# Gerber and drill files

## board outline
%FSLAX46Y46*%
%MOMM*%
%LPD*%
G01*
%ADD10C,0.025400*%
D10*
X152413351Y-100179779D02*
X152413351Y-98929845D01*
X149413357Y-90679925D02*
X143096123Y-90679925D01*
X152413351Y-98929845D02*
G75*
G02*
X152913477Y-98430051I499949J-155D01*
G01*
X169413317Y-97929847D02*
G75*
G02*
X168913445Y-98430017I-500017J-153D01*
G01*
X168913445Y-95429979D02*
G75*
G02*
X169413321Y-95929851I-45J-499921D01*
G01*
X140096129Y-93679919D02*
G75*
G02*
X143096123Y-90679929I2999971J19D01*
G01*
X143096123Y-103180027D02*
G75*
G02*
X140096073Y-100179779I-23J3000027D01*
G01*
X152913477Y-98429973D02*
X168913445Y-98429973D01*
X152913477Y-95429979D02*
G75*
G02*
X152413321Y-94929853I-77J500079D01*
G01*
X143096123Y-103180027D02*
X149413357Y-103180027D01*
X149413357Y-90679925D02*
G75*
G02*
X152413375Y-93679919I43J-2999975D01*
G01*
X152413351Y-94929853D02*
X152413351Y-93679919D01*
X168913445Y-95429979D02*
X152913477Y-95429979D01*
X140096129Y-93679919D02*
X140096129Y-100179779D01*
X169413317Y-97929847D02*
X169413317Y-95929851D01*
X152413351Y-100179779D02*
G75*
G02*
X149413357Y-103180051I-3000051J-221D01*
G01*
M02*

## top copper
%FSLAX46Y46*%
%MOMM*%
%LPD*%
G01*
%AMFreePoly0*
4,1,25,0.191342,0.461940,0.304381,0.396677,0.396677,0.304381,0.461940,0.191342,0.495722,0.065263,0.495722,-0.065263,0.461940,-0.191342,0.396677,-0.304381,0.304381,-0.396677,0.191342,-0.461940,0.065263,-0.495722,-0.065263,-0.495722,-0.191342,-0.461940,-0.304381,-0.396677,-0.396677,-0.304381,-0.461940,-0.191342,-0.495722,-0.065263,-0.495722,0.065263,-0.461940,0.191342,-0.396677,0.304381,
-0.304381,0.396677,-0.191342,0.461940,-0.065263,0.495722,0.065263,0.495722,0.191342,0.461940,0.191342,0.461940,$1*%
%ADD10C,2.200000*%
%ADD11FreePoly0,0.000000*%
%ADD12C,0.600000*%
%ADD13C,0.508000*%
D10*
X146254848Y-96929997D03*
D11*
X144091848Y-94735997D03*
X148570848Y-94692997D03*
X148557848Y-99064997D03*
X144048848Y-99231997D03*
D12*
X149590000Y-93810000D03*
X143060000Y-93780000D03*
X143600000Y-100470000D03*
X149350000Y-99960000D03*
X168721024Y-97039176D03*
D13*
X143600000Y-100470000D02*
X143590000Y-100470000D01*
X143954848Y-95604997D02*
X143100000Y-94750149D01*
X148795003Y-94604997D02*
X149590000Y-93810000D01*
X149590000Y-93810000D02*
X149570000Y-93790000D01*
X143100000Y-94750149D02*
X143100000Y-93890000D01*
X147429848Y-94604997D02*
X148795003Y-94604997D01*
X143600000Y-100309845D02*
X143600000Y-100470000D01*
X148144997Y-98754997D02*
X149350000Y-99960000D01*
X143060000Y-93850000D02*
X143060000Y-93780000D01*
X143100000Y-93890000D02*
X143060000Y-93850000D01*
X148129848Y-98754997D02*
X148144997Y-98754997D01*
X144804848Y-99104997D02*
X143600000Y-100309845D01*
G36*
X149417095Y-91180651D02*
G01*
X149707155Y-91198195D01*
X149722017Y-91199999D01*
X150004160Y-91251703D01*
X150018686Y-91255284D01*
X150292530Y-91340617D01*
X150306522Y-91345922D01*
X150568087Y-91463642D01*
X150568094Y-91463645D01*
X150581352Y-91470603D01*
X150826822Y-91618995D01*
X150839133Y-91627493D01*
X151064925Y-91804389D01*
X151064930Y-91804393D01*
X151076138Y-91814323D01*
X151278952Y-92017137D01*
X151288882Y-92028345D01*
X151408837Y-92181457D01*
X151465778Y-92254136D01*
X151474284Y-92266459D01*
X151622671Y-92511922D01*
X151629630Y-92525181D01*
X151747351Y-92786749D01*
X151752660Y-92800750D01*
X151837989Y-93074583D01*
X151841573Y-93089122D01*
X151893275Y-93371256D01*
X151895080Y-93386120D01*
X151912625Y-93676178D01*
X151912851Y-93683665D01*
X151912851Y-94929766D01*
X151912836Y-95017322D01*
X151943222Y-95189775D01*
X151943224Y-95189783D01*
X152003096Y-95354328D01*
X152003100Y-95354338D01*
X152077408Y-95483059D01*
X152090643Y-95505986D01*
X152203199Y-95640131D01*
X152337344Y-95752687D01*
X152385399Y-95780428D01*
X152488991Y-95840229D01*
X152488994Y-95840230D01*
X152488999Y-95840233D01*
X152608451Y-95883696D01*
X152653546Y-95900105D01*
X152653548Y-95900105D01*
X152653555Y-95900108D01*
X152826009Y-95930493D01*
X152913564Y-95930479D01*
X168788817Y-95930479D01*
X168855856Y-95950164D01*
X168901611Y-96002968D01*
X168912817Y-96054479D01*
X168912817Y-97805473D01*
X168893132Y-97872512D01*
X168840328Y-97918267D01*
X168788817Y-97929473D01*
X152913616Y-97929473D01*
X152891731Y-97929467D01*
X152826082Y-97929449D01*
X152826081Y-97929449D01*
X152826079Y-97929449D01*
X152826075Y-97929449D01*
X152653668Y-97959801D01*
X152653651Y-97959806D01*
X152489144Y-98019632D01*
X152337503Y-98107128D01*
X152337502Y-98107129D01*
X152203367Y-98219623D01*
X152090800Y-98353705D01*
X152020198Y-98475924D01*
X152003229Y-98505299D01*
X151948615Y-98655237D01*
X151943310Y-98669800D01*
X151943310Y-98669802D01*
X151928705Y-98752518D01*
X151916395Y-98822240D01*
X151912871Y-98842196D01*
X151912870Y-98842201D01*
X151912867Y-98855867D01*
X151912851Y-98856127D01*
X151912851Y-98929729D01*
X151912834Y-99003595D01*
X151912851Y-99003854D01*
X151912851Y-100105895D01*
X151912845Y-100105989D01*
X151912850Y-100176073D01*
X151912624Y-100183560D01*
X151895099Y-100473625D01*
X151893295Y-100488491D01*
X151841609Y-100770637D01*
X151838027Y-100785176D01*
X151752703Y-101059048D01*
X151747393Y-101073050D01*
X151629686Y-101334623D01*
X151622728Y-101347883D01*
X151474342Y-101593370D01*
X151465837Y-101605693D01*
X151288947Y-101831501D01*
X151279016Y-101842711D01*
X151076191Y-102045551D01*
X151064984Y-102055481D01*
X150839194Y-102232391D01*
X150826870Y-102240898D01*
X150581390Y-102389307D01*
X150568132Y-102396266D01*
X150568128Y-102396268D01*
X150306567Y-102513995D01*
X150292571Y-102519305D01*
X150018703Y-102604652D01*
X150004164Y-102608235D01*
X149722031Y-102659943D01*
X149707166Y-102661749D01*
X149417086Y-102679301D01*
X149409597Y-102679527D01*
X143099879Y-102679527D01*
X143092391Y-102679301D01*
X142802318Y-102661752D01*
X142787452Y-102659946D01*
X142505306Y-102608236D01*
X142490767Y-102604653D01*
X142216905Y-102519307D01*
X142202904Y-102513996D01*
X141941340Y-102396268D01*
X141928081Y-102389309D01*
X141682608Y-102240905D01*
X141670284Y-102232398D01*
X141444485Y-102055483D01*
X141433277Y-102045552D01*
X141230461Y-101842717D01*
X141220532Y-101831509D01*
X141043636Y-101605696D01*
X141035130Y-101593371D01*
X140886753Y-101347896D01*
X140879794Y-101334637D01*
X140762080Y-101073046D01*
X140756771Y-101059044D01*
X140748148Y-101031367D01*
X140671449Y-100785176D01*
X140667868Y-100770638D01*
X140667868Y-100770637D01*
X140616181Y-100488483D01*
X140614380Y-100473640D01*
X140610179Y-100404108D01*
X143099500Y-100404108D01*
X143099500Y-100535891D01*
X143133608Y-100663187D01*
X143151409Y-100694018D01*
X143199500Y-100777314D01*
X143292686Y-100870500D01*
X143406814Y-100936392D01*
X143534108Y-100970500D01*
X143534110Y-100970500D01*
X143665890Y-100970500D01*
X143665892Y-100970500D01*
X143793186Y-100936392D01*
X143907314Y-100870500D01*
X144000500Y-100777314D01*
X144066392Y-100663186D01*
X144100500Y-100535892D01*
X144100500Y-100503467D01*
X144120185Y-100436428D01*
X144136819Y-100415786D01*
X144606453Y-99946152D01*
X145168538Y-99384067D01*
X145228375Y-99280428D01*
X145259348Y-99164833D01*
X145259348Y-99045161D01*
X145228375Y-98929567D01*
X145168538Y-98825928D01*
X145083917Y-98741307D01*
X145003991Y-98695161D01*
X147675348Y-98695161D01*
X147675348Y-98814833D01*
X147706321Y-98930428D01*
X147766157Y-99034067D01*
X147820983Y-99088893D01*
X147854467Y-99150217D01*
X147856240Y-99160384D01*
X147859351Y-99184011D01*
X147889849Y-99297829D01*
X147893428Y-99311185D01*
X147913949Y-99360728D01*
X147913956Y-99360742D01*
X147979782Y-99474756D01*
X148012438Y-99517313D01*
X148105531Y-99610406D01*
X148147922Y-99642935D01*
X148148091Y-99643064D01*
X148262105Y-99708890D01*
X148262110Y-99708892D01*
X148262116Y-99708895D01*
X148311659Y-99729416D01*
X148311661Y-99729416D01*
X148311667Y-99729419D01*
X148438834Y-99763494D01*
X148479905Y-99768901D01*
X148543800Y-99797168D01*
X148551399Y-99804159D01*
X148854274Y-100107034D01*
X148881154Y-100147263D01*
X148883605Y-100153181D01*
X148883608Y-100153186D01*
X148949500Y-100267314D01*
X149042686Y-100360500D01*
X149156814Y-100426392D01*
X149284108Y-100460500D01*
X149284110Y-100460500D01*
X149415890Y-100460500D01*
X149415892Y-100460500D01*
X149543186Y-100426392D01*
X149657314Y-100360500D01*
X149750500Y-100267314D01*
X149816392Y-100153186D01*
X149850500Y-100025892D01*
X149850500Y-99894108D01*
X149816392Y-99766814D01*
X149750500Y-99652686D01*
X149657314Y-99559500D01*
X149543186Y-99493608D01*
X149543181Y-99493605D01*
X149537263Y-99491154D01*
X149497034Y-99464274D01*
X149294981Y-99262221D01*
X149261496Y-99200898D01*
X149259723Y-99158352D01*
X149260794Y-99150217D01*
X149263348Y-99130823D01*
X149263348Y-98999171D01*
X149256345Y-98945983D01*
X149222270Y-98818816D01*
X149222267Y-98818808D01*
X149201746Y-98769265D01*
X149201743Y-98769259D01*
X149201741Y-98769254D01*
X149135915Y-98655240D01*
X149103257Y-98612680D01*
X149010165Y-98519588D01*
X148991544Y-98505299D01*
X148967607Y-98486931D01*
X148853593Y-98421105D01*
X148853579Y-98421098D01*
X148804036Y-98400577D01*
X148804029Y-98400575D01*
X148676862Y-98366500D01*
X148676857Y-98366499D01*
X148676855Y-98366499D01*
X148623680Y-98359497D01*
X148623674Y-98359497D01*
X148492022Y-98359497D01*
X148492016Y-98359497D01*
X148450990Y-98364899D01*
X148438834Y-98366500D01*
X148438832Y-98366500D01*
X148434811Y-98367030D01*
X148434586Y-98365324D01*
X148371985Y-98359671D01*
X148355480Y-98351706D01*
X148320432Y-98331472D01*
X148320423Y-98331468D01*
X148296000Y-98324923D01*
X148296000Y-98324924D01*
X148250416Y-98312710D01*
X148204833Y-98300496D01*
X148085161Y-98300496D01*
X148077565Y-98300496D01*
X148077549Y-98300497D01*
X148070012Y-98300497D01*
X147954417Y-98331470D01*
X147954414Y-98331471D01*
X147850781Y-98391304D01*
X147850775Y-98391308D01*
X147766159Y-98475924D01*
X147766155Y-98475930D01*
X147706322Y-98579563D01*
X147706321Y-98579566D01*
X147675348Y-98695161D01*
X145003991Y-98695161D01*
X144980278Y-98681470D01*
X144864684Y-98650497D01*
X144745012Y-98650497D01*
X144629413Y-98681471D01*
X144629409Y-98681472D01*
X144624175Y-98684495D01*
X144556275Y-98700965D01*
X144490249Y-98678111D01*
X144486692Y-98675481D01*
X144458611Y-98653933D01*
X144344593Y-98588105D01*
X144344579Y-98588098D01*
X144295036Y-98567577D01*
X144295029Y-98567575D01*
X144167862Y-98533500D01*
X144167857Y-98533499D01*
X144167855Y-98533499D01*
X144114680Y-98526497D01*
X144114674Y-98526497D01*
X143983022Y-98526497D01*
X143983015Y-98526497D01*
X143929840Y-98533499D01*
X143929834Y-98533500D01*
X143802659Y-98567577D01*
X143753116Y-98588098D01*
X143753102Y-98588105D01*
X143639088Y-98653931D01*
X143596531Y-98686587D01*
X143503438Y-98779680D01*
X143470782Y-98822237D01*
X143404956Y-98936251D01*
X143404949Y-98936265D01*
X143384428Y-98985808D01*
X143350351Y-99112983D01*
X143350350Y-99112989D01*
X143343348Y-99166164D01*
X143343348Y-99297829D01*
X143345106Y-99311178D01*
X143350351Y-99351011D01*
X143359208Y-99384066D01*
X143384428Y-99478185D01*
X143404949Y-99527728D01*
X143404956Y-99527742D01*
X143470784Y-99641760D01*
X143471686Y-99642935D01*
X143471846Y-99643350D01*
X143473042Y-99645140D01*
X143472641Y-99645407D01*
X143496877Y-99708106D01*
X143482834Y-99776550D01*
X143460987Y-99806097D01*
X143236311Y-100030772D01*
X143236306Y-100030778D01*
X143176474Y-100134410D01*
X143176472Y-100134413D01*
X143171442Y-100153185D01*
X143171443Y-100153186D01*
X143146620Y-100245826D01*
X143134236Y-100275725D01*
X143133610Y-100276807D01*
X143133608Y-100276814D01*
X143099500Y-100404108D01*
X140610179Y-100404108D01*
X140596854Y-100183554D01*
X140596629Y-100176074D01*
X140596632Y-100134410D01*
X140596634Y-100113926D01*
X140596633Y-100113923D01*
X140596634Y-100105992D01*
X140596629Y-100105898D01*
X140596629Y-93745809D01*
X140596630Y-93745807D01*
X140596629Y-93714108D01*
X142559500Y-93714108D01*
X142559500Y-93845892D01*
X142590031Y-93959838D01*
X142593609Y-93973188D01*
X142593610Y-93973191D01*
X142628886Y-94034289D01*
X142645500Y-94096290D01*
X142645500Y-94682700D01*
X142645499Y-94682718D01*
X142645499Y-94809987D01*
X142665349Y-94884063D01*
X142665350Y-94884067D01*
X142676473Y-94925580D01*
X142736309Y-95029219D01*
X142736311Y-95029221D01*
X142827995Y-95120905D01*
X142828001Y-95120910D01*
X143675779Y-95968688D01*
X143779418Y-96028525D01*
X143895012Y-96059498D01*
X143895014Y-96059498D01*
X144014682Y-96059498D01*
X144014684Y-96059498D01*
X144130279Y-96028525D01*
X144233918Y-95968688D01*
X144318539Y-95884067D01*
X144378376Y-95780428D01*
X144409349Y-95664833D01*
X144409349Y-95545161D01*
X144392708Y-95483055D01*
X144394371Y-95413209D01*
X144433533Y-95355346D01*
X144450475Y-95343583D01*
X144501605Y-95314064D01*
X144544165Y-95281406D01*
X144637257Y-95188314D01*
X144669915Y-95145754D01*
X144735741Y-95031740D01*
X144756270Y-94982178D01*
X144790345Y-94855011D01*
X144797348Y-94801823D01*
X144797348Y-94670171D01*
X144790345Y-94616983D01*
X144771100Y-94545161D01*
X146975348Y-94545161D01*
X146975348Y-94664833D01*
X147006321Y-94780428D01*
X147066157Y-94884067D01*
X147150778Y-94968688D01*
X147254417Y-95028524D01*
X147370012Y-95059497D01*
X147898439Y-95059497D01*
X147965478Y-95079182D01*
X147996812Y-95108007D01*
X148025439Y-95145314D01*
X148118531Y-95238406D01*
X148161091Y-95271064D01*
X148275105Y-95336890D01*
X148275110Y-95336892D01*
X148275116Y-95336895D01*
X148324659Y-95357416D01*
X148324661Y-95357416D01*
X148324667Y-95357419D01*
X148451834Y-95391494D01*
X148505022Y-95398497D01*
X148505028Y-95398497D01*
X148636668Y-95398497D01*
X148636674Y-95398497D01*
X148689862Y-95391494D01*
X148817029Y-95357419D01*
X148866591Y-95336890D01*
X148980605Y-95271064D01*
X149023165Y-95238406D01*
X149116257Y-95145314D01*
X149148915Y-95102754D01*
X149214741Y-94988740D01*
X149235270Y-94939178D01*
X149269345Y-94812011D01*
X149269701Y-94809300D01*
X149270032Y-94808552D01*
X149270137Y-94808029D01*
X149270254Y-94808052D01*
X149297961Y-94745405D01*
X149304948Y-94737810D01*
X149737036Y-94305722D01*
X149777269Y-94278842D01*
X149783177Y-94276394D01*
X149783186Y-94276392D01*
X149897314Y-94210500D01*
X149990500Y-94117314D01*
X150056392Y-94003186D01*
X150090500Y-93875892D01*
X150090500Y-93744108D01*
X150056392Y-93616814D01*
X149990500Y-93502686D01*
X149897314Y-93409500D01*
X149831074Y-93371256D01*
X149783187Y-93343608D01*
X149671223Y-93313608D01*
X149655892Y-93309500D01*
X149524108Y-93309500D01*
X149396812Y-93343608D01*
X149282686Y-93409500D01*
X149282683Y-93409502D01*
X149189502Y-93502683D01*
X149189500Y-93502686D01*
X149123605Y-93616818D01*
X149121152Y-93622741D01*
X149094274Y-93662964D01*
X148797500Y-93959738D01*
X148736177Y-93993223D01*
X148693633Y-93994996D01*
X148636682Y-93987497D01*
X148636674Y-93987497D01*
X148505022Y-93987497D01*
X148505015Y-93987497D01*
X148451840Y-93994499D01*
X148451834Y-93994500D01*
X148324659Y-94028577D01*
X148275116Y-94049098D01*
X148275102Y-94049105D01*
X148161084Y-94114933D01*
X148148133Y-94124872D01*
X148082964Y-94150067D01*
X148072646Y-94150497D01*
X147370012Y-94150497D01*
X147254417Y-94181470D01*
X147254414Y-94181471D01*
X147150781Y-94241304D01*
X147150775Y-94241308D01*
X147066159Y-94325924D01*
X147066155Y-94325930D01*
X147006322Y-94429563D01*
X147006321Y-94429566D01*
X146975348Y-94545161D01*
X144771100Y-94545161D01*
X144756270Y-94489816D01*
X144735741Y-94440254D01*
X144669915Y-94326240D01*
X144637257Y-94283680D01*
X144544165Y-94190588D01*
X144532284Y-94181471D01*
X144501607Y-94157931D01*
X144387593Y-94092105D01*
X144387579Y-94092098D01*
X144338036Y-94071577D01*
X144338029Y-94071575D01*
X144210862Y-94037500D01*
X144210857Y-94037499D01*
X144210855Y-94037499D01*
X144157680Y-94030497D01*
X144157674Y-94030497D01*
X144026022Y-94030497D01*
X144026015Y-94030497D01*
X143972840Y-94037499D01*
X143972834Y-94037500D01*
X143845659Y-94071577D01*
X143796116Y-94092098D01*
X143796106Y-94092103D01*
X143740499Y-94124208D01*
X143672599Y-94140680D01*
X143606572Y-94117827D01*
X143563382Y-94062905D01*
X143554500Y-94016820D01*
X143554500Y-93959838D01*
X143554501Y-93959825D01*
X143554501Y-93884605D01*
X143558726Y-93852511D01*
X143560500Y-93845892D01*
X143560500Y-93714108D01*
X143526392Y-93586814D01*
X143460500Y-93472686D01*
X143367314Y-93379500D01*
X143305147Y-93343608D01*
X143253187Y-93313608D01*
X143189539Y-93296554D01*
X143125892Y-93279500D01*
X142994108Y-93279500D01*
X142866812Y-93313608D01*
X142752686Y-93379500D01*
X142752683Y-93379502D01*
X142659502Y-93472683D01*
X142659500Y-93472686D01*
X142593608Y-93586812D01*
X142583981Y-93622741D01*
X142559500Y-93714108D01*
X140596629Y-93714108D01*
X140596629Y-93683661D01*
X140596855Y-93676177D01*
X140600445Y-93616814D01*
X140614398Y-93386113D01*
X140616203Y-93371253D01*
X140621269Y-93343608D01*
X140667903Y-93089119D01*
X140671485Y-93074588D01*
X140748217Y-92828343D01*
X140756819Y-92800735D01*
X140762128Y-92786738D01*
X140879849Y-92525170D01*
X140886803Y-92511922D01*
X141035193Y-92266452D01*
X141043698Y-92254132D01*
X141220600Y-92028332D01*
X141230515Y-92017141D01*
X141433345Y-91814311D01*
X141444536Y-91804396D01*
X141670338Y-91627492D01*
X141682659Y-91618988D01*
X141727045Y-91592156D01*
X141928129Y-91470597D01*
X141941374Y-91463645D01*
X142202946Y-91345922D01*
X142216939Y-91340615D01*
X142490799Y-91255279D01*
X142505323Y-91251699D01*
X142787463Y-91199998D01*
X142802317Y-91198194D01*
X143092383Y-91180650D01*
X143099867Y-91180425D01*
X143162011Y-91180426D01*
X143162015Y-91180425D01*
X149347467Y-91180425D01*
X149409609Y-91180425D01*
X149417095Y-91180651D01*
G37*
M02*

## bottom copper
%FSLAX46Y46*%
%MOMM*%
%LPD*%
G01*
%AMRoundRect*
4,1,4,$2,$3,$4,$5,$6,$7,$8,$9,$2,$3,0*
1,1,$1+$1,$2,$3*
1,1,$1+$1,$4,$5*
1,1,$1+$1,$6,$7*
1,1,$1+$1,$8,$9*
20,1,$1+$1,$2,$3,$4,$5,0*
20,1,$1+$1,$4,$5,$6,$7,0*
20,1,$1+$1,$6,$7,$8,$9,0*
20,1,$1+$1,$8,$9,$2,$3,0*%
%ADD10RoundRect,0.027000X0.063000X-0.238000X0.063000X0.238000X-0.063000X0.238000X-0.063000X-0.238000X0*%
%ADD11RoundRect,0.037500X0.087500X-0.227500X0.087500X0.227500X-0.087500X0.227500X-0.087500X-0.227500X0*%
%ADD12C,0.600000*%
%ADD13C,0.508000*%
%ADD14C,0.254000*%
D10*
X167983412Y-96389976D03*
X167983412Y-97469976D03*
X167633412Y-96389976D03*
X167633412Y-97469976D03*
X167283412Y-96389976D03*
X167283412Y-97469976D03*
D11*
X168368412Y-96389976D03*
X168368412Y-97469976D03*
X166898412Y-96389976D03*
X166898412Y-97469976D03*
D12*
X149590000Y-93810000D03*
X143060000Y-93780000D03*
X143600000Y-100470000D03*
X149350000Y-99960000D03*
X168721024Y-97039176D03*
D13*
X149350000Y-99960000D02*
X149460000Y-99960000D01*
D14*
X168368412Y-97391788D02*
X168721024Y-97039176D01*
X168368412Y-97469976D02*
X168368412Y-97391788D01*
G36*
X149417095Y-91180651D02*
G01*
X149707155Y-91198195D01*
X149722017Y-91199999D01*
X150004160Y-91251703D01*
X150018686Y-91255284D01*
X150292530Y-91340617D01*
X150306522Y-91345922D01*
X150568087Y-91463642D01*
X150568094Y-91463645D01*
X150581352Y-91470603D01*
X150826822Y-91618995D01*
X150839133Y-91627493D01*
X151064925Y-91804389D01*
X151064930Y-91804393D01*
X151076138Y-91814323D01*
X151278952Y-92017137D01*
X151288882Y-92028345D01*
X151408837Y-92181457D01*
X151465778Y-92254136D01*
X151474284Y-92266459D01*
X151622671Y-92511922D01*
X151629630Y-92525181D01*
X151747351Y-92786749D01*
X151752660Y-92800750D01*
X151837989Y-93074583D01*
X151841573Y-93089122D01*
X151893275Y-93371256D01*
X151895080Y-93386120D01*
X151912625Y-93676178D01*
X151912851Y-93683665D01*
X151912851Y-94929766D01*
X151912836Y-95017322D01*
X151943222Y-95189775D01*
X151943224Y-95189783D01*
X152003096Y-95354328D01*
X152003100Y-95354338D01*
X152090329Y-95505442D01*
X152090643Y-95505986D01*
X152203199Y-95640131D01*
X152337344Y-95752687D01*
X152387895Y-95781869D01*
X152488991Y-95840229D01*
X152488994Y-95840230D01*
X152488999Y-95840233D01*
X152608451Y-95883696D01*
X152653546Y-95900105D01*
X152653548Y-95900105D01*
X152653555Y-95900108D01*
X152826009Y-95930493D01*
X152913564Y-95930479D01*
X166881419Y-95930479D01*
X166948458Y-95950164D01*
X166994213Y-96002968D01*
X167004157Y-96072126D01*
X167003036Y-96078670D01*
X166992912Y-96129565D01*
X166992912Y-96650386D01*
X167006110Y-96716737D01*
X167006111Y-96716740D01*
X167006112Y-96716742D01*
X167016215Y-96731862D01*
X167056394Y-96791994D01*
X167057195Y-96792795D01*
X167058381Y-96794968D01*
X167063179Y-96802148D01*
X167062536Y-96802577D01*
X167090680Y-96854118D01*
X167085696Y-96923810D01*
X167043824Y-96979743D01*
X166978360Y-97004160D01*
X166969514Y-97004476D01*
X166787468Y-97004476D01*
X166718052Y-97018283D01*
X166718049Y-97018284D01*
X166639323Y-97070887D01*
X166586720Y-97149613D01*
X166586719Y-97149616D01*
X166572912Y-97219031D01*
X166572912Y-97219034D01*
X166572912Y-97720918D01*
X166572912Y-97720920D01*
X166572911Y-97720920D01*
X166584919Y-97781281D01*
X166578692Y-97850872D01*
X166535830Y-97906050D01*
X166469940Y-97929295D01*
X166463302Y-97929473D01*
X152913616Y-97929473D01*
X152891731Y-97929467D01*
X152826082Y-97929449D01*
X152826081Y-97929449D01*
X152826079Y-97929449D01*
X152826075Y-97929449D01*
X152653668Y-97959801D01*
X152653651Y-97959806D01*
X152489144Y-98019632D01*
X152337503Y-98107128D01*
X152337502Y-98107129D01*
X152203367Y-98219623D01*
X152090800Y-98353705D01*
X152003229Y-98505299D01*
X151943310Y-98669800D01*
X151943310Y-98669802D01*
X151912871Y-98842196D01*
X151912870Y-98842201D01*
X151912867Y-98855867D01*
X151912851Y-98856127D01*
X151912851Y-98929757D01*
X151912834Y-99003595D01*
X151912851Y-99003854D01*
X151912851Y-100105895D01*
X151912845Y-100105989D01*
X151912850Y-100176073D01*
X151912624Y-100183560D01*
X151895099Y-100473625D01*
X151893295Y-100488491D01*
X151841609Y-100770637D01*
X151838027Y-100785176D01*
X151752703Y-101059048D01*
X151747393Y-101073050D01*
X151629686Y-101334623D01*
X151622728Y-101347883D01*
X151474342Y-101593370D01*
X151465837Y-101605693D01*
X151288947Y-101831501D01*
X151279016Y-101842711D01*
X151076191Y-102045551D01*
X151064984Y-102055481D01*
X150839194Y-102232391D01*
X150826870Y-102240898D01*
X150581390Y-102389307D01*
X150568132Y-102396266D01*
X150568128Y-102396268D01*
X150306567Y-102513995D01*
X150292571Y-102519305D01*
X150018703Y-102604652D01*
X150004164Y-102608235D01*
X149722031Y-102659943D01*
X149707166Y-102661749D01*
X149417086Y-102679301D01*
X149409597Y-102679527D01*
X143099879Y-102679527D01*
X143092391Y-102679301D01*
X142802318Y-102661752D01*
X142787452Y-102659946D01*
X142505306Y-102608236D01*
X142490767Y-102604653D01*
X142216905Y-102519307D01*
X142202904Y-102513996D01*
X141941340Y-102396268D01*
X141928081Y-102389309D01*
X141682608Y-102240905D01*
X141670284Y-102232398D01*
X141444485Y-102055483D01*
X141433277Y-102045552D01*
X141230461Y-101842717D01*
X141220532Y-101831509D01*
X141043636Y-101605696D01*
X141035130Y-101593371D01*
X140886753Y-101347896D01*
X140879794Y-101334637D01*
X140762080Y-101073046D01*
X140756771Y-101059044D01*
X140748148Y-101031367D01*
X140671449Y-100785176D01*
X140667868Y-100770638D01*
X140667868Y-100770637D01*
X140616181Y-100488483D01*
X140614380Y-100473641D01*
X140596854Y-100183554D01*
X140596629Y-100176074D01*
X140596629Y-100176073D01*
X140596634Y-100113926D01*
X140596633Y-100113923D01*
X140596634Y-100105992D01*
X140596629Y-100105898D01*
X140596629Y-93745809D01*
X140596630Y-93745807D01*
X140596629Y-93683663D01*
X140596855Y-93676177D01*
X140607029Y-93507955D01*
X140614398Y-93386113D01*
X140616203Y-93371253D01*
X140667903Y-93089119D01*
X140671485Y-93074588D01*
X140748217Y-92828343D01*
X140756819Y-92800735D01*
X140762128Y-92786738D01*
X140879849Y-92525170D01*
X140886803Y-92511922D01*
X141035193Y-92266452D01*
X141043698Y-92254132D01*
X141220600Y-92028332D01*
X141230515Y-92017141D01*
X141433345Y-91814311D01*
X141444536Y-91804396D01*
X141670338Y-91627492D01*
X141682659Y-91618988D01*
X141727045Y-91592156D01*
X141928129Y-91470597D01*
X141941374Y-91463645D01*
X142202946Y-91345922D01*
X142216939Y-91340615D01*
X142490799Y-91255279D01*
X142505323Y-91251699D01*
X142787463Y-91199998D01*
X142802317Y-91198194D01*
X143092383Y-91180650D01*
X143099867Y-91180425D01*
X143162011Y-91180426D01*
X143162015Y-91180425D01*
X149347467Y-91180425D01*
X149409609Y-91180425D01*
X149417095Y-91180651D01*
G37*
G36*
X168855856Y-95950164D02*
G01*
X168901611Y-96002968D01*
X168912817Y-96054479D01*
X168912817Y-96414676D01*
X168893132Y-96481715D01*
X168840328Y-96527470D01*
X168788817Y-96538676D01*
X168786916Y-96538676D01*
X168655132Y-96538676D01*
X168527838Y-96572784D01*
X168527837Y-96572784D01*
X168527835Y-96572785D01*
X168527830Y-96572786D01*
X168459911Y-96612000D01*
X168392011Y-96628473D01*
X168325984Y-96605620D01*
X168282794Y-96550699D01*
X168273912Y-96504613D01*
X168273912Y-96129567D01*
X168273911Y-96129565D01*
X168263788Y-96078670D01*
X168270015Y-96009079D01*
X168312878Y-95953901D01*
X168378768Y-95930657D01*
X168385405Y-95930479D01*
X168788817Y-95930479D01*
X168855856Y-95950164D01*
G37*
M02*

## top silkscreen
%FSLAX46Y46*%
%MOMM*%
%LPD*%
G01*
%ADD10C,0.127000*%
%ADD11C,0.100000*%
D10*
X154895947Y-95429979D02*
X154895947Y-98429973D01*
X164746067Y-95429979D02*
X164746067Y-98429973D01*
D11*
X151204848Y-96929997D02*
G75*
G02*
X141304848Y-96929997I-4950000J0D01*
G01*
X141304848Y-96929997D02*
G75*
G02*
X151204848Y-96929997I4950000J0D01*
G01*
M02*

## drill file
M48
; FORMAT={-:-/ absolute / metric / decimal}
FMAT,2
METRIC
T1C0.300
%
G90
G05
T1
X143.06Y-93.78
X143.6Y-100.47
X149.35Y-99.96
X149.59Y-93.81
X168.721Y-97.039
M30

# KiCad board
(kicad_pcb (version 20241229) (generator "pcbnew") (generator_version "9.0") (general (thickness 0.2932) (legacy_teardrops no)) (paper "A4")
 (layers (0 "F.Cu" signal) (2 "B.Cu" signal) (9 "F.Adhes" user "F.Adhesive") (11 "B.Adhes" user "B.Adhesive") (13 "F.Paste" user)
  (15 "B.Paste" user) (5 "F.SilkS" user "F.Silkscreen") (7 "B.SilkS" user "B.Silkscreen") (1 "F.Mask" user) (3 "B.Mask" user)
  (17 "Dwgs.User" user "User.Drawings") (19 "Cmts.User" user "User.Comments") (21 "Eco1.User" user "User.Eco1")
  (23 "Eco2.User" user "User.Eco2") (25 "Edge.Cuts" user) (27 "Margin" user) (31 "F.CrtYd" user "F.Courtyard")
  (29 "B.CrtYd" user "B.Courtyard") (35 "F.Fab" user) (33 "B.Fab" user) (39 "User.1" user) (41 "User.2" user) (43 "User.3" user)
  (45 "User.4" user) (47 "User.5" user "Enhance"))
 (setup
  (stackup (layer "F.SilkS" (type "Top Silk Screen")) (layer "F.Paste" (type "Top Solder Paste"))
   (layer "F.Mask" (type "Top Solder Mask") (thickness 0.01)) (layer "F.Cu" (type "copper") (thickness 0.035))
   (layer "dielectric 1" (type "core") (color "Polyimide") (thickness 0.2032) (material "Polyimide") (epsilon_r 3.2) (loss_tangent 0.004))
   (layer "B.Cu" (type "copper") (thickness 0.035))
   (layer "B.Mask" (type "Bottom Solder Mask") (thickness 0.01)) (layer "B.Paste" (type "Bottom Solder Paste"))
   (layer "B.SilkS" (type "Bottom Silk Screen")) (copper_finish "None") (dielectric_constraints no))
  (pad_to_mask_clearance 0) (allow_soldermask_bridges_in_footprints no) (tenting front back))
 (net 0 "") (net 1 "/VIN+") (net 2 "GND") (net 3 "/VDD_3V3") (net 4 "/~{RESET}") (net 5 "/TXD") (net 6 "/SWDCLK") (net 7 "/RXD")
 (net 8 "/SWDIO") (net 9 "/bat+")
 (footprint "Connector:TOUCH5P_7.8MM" (layer "F.Cu") (at 146.254848 96.929997)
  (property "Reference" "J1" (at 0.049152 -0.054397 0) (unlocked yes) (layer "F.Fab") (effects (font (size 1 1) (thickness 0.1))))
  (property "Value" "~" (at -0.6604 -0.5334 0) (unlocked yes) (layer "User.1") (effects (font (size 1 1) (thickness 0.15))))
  (fp_circle (center 0 0) (end 4.95 0) (stroke (width 0.1) (type default)) (fill no) (layer "F.SilkS"))
  (pad "1" smd circle (at 0 0) (size 2.2 2.2) (layers "F.Cu" "F.Mask" "F.Paste") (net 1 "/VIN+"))
  (pad "2" smd custom (at -2.163 -2.194) (size 1 1) (layers "F.Cu" "F.Mask" "F.Paste") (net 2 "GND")
   (options (clearance outline) (anchor circle)) (primitives))
  (pad "3" smd custom (at 2.316 -2.237) (size 1 2.2) (layers "F.Cu" "F.Mask" "F.Paste") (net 2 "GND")
   (options (clearance outline) (anchor circle)) (primitives))
  (pad "4" smd custom (at 2.303 2.135) (size 1 1) (layers "F.Cu" "F.Mask" "F.Paste") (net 2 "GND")
   (options (clearance outline) (anchor circle)) (primitives))
  (pad "5" smd custom (at -2.206 2.302) (size 1 1) (layers "F.Cu" "F.Mask" "F.Paste") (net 2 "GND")
   (options (clearance outline) (anchor circle)) (primitives)))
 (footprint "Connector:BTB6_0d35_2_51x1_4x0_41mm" (layer "B.Cu") (at 167.633412 96.929976 180)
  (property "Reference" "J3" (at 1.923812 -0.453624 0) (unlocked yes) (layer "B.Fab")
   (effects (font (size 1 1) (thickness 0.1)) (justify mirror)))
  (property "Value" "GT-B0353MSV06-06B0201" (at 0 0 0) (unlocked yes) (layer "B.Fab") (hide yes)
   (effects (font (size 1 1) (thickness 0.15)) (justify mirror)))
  (pad "1" smd roundrect (at -0.35 0.54 90) (size 0.53 0.18) (layers "B.Cu" "B.Mask" "B.Paste") (roundrect_rratio 0.15) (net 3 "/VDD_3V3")
   (thermal_bridge_angle 45))
  (pad "2" smd roundrect (at -0.35 -0.54 90) (size 0.53 0.18) (layers "B.Cu" "B.Mask" "B.Paste") (roundrect_rratio 0.15) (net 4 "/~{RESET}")
   (thermal_bridge_angle 45))
  (pad "3" smd roundrect (at 0 0.54 90) (size 0.53 0.18) (layers "B.Cu" "B.Mask" "B.Paste") (roundrect_rratio 0.15) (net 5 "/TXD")
   (thermal_bridge_angle 45))
  (pad "4" smd roundrect (at 0 -0.54 90) (size 0.53 0.18) (layers "B.Cu" "B.Mask" "B.Paste") (roundrect_rratio 0.15) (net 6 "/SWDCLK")
   (thermal_bridge_angle 45))
  (pad "5" smd roundrect (at 0.35 0.54 90) (size 0.53 0.18) (layers "B.Cu" "B.Mask" "B.Paste") (roundrect_rratio 0.15) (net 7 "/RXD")
   (thermal_bridge_angle 45))
  (pad "6" smd roundrect (at 0.35 -0.54 90) (size 0.53 0.18) (layers "B.Cu" "B.Mask" "B.Paste") (roundrect_rratio 0.15) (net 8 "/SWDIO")
   (thermal_bridge_angle 45))
  (pad "S1" smd roundrect (at -0.735 0.54 90) (size 0.53 0.25) (layers "B.Cu" "B.Mask" "B.Paste") (roundrect_rratio 0.15) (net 2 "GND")
   (thermal_bridge_angle 45))
  (pad "S2" smd roundrect (at -0.735 -0.54 90) (size 0.53 0.25) (layers "B.Cu" "B.Mask" "B.Paste") (roundrect_rratio 0.15) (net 1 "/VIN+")
   (thermal_bridge_angle 45))
  (pad "S3" smd roundrect (at 0.735 0.54 90) (size 0.53 0.25) (layers "B.Cu" "B.Mask" "B.Paste") (roundrect_rratio 0.15) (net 2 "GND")
   (thermal_bridge_angle 45))
  (pad "S4" smd roundrect (at 0.735 -0.54 90) (size 0.53 0.25) (layers "B.Cu" "B.Mask" "B.Paste") (roundrect_rratio 0.15) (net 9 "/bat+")
   (thermal_bridge_angle 45)))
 (gr_line (start 154.895947 95.429979) (end 154.895947 98.429973) (stroke (width 0.127) (type default)) (layer "F.SilkS"))
 (gr_line (start 164.746067 95.429979) (end 164.746067 98.429973) (stroke (width 0.127) (type default)) (layer "F.SilkS"))
 (gr_line (start 152.413351 100.179779) (end 152.413351 98.929845) (stroke (width 0.0254) (type default)) (layer "Edge.Cuts"))
 (gr_line (start 149.413357 90.679925) (end 143.096123 90.679925) (stroke (width 0.0254) (type default)) (layer "Edge.Cuts"))
 (gr_arc (start 152.413351 98.929845) (mid 152.559884 98.576326) (end 152.913477 98.429973) (stroke (width 0.0254) (type default))
  (layer "Edge.Cuts"))
 (gr_arc (start 169.413317 97.929847) (mid 169.26696 98.283436) (end 168.913445 98.429973) (stroke (width 0.0254) (type default))
  (layer "Edge.Cuts"))
 (gr_arc (start 168.913445 95.429979) (mid 169.266885 95.576411) (end 169.413317 95.929851) (stroke (width 0.0254) (type default))
  (layer "Edge.Cuts"))
 (gr_arc (start 140.096129 93.679919) (mid 140.974799 91.558595) (end 143.096123 90.679925) (stroke (width 0.0254) (type default))
  (layer "Edge.Cuts"))
 (gr_arc (start 143.096123 103.180027) (mid 140.974724 102.301253) (end 140.096129 100.179779) (stroke (width 0.0254) (type default))
  (layer "Edge.Cuts"))
 (gr_line (start 152.913477 98.429973) (end 168.913445 98.429973) (stroke (width 0.0254) (type default)) (layer "Edge.Cuts"))
 (gr_arc (start 152.913477 95.429979) (mid 152.559809 95.283521) (end 152.413351 94.929853) (stroke (width 0.0254) (type default))
  (layer "Edge.Cuts"))
 (gr_line (start 143.096123 103.180027) (end 149.413357 103.180027) (stroke (width 0.0254) (type default)) (layer "Edge.Cuts"))
 (gr_arc (start 149.413357 90.679925) (mid 151.534677 91.558599) (end 152.413351 93.679919) (stroke (width 0.0254) (type default))
  (layer "Edge.Cuts"))
 (gr_line (start 152.413351 94.929853) (end 152.413351 93.679919) (stroke (width 0.0254) (type default)) (layer "Edge.Cuts"))
 (gr_line (start 168.913445 95.429979) (end 152.913477 95.429979) (stroke (width 0.0254) (type default)) (layer "Edge.Cuts"))
 (gr_line (start 140.096129 93.679919) (end 140.096129 100.179779) (stroke (width 0.0254) (type default)) (layer "Edge.Cuts"))
 (gr_line (start 169.413317 97.929847) (end 169.413317 95.929851) (stroke (width 0.0254) (type default)) (layer "Edge.Cuts"))
 (gr_arc (start 152.413351 100.179779) (mid 151.534752 102.301248) (end 149.413357 103.180027) (stroke (width 0.0254) (type default))
  (layer "Edge.Cuts"))
 (segment (start 143.6 100.47) (end 143.59 100.47) (width 0.508) (layer "F.Cu") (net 2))
 (segment (start 143.954848 95.604997) (end 143.1 94.750149) (width 0.508) (layer "F.Cu") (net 2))
 (segment (start 148.795003 94.604997) (end 149.59 93.81) (width 0.508) (layer "F.Cu") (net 2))
 (segment (start 149.59 93.81) (end 149.57 93.79) (width 0.508) (layer "F.Cu") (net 2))
 (segment (start 143.1 94.750149) (end 143.1 93.89) (width 0.508) (layer "F.Cu") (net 2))
 (segment (start 147.429848 94.604997) (end 148.795003 94.604997) (width 0.508) (layer "F.Cu") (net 2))
 (segment (start 143.6 100.309845) (end 143.6 100.47) (width 0.508) (layer "F.Cu") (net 2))
 (segment (start 148.144997 98.754997) (end 149.35 99.96) (width 0.508) (layer "F.Cu") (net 2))
 (segment (start 143.06 93.85) (end 143.06 93.78) (width 0.508) (layer "F.Cu") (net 2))
 (segment (start 143.1 93.89) (end 143.06 93.85) (width 0.508) (layer "F.Cu") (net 2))
 (segment (start 148.129848 98.754997) (end 148.144997 98.754997) (width 0.508) (layer "F.Cu") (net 2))
 (segment (start 144.804848 99.104997) (end 143.6 100.309845) (width 0.508) (layer "F.Cu") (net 2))
 (via (at 149.59 93.81) (size 0.6) (drill 0.3) (layers "F.Cu" "B.Cu") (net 2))
 (via (at 143.06 93.78) (size 0.6) (drill 0.3) (layers "F.Cu" "B.Cu") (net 2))
 (via (at 143.6 100.47) (size 0.6) (drill 0.3) (layers "F.Cu" "B.Cu") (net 2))
 (via (at 149.35 99.96) (size 0.6) (drill 0.3) (layers "F.Cu" "B.Cu") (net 2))
 (segment (start 149.35 99.96) (end 149.46 99.96) (width 0.508) (layer "B.Cu") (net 2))
 (via (at 168.721024 97.039176) (size 0.6) (drill 0.3) (layers "F.Cu" "B.Cu") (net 1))
 (segment (start 168.368412 97.391788) (end 168.721024 97.039176) (width 0.254) (layer "B.Cu") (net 1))
 (segment (start 168.368412 97.469976) (end 168.368412 97.391788) (width 0.254) (layer "B.Cu") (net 1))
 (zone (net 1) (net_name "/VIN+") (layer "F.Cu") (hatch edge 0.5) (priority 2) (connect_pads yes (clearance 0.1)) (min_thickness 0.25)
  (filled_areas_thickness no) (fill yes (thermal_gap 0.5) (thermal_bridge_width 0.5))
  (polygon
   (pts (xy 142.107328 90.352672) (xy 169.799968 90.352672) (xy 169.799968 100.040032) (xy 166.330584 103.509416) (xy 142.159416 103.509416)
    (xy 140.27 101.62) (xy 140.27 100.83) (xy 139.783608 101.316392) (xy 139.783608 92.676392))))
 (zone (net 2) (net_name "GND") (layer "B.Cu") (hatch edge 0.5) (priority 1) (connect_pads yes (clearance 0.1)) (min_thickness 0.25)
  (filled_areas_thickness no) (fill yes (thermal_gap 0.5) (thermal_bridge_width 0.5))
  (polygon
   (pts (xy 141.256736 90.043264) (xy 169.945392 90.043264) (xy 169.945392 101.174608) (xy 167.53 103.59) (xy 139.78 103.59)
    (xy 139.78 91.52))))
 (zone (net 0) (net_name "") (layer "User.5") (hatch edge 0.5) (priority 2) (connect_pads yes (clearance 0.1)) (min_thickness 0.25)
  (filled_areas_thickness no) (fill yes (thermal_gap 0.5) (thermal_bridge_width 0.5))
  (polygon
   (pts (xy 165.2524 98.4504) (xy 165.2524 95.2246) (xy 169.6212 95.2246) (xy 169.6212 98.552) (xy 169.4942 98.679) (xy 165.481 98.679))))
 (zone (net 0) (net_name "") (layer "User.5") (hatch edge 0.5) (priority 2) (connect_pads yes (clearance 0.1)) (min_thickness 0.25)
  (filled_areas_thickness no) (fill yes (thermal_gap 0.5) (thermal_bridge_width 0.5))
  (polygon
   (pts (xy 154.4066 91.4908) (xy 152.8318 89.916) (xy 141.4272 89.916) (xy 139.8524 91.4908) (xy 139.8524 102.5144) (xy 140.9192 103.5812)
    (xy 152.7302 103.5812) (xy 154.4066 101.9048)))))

